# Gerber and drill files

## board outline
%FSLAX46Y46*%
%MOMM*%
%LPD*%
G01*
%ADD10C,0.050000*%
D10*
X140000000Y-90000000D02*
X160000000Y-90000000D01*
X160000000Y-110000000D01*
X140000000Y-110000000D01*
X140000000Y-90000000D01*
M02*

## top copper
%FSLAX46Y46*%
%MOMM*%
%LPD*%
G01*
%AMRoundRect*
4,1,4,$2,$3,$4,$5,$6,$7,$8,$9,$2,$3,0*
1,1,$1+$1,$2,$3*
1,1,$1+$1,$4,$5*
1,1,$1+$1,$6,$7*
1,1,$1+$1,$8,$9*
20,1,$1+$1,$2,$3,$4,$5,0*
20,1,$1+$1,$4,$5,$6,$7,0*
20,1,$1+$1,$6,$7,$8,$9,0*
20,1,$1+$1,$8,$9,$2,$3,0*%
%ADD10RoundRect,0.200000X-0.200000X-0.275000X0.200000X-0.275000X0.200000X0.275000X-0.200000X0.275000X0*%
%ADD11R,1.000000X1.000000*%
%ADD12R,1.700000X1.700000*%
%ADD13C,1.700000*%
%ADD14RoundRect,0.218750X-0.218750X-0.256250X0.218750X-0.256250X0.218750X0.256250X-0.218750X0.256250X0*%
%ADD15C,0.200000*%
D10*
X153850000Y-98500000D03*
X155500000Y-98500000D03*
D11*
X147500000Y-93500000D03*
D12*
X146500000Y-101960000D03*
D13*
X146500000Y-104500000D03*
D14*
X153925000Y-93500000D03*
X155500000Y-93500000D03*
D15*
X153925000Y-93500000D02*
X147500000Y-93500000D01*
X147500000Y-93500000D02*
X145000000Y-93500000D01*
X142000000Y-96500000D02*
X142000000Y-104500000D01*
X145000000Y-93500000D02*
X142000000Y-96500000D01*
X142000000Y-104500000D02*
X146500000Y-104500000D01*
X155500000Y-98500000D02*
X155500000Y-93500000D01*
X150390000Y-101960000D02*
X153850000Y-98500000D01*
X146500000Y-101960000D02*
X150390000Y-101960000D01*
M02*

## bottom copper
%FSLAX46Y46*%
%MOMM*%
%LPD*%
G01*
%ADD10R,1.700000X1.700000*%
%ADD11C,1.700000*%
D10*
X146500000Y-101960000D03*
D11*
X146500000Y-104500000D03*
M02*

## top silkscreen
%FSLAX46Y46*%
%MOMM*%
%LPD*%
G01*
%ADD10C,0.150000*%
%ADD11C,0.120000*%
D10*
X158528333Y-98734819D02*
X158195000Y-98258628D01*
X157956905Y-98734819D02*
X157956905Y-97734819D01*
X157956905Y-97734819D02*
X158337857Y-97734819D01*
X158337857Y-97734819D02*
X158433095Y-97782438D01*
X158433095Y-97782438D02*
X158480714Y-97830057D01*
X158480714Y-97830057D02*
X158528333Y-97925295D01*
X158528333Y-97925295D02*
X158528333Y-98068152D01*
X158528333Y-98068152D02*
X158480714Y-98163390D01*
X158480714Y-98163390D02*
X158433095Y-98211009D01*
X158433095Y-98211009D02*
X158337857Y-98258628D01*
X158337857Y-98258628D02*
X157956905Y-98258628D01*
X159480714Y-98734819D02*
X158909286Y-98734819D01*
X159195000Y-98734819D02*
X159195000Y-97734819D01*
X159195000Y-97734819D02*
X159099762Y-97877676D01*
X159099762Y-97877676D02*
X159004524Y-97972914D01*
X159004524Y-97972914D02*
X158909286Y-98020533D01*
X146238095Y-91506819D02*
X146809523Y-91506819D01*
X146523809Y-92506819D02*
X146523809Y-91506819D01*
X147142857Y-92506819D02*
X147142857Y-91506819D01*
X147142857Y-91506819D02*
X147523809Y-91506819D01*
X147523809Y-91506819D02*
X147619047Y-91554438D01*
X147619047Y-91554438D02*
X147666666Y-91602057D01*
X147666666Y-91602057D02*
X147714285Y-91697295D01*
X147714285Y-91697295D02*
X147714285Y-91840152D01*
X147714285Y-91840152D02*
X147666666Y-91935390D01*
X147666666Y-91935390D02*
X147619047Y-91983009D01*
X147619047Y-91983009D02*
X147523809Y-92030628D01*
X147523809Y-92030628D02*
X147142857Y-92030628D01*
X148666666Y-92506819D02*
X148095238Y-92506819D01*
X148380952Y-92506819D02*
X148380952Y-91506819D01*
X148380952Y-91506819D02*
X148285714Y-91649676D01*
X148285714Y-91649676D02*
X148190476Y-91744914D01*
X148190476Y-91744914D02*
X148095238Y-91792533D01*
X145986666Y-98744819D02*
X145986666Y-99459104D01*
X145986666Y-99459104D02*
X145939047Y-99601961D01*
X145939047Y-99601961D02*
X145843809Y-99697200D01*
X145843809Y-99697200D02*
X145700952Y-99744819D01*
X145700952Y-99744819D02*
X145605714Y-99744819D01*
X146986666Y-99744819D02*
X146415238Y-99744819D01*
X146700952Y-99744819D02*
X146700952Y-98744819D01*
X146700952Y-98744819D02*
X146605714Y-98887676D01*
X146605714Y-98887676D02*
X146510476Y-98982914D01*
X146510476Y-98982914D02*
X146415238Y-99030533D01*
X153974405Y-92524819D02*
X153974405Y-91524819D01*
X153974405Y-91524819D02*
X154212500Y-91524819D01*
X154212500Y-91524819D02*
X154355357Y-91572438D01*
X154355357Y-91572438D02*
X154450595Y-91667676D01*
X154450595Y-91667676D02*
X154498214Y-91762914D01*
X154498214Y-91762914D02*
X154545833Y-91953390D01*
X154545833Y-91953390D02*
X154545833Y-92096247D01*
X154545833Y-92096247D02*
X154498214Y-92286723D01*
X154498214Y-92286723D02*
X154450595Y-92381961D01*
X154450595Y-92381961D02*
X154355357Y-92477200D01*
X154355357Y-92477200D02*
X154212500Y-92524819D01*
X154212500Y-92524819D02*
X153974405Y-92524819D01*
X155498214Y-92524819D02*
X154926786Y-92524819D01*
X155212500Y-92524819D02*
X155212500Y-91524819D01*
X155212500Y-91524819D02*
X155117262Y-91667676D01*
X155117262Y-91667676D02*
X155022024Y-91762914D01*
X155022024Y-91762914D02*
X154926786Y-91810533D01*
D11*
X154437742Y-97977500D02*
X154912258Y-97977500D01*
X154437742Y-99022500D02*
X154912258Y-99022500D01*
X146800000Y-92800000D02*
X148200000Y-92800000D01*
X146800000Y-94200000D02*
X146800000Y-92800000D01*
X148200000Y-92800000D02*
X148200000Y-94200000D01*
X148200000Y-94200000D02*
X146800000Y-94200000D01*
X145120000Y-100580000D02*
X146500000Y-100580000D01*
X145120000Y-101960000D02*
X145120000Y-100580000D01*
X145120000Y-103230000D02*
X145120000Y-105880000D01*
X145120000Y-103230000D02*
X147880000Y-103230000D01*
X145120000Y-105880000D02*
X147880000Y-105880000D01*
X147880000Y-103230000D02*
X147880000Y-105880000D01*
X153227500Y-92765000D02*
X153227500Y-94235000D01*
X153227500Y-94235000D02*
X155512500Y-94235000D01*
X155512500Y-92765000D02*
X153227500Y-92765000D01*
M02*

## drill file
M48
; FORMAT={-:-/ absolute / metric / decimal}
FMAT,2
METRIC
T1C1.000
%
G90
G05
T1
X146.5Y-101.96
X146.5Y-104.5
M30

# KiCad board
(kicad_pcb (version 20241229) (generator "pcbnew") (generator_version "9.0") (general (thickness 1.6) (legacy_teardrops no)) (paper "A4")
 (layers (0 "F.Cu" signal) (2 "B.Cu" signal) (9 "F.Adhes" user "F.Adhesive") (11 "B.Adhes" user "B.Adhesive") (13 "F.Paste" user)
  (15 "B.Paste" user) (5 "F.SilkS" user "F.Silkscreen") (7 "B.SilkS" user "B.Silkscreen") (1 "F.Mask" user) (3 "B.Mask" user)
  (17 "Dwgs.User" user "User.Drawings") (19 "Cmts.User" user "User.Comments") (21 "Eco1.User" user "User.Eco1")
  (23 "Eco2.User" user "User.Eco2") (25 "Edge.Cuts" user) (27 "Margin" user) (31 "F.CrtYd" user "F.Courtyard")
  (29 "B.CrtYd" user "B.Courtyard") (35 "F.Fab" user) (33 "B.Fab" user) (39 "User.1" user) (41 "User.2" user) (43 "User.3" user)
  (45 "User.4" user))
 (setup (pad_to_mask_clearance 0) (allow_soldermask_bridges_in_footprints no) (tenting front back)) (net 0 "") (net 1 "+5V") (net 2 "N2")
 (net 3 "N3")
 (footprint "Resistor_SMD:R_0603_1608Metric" (layer "F.Cu") (at 154.675 98.5)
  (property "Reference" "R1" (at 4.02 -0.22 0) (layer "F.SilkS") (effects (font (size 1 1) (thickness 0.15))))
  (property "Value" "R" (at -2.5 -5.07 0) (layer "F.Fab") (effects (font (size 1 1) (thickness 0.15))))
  (fp_line (start -0.237258 -0.5225) (end 0.237258 -0.5225) (stroke (width 0.12) (type solid)) (layer "F.SilkS"))
  (fp_line (start -0.237258 0.5225) (end 0.237258 0.5225) (stroke (width 0.12) (type solid)) (layer "F.SilkS"))
  (pad "1" smd roundrect (at -0.825 0) (size 0.8 0.95) (layers "F.Cu" "F.Mask" "F.Paste") (roundrect_rratio 0.25) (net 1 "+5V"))
  (pad "2" smd roundrect (at 0.825 0) (size 0.8 0.95) (layers "F.Cu" "F.Mask" "F.Paste") (roundrect_rratio 0.25) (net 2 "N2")))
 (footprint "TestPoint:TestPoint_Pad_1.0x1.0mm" (layer "F.Cu") (at 147.5 93.5)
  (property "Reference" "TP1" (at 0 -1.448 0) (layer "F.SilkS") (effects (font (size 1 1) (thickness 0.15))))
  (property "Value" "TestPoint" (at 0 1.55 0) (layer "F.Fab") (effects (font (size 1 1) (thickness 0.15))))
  (fp_line (start -0.7 -0.7) (end 0.7 -0.7) (stroke (width 0.12) (type solid)) (layer "F.SilkS"))
  (fp_line (start -0.7 0.7) (end -0.7 -0.7) (stroke (width 0.12) (type solid)) (layer "F.SilkS"))
  (fp_line (start 0.7 -0.7) (end 0.7 0.7) (stroke (width 0.12) (type solid)) (layer "F.SilkS"))
  (fp_line (start 0.7 0.7) (end -0.7 0.7) (stroke (width 0.12) (type solid)) (layer "F.SilkS"))
  (pad "1" smd rect (at 0 0) (size 1 1) (layers "F.Cu" "F.Mask") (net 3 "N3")))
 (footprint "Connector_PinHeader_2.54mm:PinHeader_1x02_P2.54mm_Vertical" (layer "F.Cu") (at 146.5 101.96)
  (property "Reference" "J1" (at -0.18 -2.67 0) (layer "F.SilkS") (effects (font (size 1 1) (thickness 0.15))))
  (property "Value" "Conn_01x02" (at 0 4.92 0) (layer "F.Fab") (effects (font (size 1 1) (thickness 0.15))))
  (fp_line (start -1.38 -1.38) (end 0 -1.38) (stroke (width 0.12) (type solid)) (layer "F.SilkS"))
  (fp_line (start -1.38 0) (end -1.38 -1.38) (stroke (width 0.12) (type solid)) (layer "F.SilkS"))
  (fp_line (start -1.38 1.27) (end -1.38 3.92) (stroke (width 0.12) (type solid)) (layer "F.SilkS"))
  (fp_line (start -1.38 1.27) (end 1.38 1.27) (stroke (width 0.12) (type solid)) (layer "F.SilkS"))
  (fp_line (start -1.38 3.92) (end 1.38 3.92) (stroke (width 0.12) (type solid)) (layer "F.SilkS"))
  (fp_line (start 1.38 1.27) (end 1.38 3.92) (stroke (width 0.12) (type solid)) (layer "F.SilkS"))
  (pad "1" thru_hole rect (at 0 0) (size 1.7 1.7) (drill 1) (layers "*.Cu" "*.Mask") (remove_unused_layers no) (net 1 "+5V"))
  (pad "2" thru_hole circle (at 0 2.54) (size 1.7 1.7) (drill 1) (layers "*.Cu" "*.Mask") (remove_unused_layers no) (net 3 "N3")))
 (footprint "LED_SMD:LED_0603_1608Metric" (layer "F.Cu") (at 154.7125 93.5)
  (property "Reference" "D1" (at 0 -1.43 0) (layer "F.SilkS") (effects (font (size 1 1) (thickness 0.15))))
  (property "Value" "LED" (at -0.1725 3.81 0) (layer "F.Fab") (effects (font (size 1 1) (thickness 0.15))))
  (fp_line (start -1.485 -0.735) (end -1.485 0.735) (stroke (width 0.12) (type solid)) (layer "F.SilkS"))
  (fp_line (start -1.485 0.735) (end 0.8 0.735) (stroke (width 0.12) (type solid)) (layer "F.SilkS"))
  (fp_line (start 0.8 -0.735) (end -1.485 -0.735) (stroke (width 0.12) (type solid)) (layer "F.SilkS"))
  (pad "1" smd roundrect (at -0.7875 0) (size 0.875 0.95) (layers "F.Cu" "F.Mask" "F.Paste") (roundrect_rratio 0.25) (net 3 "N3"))
  (pad "2" smd roundrect (at 0.7875 0) (size 0.875 0.95) (layers "F.Cu" "F.Mask" "F.Paste") (roundrect_rratio 0.25) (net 2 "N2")))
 (gr_rect (start 140 90) (end 160 110) (stroke (width 0.05) (type default)) (fill no) (layer "Edge.Cuts"))
 (segment (start 153.925 93.5) (end 147.5 93.5) (width 0.2) (layer "F.Cu") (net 3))
 (segment (start 147.5 93.5) (end 145 93.5) (width 0.2) (layer "F.Cu") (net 3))
 (segment (start 142 96.5) (end 142 104.5) (width 0.2) (layer "F.Cu") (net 3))
 (segment (start 145 93.5) (end 142 96.5) (width 0.2) (layer "F.Cu") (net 3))
 (segment (start 142 104.5) (end 146.5 104.5) (width 0.2) (layer "F.Cu") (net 3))
 (segment (start 155.5 98.5) (end 155.5 93.5) (width 0.2) (layer "F.Cu") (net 2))
 (segment (start 150.39 101.96) (end 153.85 98.5) (width 0.2) (layer "F.Cu") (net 1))
 (segment (start 146.5 101.96) (end 150.39 101.96) (width 0.2) (layer "F.Cu") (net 1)))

